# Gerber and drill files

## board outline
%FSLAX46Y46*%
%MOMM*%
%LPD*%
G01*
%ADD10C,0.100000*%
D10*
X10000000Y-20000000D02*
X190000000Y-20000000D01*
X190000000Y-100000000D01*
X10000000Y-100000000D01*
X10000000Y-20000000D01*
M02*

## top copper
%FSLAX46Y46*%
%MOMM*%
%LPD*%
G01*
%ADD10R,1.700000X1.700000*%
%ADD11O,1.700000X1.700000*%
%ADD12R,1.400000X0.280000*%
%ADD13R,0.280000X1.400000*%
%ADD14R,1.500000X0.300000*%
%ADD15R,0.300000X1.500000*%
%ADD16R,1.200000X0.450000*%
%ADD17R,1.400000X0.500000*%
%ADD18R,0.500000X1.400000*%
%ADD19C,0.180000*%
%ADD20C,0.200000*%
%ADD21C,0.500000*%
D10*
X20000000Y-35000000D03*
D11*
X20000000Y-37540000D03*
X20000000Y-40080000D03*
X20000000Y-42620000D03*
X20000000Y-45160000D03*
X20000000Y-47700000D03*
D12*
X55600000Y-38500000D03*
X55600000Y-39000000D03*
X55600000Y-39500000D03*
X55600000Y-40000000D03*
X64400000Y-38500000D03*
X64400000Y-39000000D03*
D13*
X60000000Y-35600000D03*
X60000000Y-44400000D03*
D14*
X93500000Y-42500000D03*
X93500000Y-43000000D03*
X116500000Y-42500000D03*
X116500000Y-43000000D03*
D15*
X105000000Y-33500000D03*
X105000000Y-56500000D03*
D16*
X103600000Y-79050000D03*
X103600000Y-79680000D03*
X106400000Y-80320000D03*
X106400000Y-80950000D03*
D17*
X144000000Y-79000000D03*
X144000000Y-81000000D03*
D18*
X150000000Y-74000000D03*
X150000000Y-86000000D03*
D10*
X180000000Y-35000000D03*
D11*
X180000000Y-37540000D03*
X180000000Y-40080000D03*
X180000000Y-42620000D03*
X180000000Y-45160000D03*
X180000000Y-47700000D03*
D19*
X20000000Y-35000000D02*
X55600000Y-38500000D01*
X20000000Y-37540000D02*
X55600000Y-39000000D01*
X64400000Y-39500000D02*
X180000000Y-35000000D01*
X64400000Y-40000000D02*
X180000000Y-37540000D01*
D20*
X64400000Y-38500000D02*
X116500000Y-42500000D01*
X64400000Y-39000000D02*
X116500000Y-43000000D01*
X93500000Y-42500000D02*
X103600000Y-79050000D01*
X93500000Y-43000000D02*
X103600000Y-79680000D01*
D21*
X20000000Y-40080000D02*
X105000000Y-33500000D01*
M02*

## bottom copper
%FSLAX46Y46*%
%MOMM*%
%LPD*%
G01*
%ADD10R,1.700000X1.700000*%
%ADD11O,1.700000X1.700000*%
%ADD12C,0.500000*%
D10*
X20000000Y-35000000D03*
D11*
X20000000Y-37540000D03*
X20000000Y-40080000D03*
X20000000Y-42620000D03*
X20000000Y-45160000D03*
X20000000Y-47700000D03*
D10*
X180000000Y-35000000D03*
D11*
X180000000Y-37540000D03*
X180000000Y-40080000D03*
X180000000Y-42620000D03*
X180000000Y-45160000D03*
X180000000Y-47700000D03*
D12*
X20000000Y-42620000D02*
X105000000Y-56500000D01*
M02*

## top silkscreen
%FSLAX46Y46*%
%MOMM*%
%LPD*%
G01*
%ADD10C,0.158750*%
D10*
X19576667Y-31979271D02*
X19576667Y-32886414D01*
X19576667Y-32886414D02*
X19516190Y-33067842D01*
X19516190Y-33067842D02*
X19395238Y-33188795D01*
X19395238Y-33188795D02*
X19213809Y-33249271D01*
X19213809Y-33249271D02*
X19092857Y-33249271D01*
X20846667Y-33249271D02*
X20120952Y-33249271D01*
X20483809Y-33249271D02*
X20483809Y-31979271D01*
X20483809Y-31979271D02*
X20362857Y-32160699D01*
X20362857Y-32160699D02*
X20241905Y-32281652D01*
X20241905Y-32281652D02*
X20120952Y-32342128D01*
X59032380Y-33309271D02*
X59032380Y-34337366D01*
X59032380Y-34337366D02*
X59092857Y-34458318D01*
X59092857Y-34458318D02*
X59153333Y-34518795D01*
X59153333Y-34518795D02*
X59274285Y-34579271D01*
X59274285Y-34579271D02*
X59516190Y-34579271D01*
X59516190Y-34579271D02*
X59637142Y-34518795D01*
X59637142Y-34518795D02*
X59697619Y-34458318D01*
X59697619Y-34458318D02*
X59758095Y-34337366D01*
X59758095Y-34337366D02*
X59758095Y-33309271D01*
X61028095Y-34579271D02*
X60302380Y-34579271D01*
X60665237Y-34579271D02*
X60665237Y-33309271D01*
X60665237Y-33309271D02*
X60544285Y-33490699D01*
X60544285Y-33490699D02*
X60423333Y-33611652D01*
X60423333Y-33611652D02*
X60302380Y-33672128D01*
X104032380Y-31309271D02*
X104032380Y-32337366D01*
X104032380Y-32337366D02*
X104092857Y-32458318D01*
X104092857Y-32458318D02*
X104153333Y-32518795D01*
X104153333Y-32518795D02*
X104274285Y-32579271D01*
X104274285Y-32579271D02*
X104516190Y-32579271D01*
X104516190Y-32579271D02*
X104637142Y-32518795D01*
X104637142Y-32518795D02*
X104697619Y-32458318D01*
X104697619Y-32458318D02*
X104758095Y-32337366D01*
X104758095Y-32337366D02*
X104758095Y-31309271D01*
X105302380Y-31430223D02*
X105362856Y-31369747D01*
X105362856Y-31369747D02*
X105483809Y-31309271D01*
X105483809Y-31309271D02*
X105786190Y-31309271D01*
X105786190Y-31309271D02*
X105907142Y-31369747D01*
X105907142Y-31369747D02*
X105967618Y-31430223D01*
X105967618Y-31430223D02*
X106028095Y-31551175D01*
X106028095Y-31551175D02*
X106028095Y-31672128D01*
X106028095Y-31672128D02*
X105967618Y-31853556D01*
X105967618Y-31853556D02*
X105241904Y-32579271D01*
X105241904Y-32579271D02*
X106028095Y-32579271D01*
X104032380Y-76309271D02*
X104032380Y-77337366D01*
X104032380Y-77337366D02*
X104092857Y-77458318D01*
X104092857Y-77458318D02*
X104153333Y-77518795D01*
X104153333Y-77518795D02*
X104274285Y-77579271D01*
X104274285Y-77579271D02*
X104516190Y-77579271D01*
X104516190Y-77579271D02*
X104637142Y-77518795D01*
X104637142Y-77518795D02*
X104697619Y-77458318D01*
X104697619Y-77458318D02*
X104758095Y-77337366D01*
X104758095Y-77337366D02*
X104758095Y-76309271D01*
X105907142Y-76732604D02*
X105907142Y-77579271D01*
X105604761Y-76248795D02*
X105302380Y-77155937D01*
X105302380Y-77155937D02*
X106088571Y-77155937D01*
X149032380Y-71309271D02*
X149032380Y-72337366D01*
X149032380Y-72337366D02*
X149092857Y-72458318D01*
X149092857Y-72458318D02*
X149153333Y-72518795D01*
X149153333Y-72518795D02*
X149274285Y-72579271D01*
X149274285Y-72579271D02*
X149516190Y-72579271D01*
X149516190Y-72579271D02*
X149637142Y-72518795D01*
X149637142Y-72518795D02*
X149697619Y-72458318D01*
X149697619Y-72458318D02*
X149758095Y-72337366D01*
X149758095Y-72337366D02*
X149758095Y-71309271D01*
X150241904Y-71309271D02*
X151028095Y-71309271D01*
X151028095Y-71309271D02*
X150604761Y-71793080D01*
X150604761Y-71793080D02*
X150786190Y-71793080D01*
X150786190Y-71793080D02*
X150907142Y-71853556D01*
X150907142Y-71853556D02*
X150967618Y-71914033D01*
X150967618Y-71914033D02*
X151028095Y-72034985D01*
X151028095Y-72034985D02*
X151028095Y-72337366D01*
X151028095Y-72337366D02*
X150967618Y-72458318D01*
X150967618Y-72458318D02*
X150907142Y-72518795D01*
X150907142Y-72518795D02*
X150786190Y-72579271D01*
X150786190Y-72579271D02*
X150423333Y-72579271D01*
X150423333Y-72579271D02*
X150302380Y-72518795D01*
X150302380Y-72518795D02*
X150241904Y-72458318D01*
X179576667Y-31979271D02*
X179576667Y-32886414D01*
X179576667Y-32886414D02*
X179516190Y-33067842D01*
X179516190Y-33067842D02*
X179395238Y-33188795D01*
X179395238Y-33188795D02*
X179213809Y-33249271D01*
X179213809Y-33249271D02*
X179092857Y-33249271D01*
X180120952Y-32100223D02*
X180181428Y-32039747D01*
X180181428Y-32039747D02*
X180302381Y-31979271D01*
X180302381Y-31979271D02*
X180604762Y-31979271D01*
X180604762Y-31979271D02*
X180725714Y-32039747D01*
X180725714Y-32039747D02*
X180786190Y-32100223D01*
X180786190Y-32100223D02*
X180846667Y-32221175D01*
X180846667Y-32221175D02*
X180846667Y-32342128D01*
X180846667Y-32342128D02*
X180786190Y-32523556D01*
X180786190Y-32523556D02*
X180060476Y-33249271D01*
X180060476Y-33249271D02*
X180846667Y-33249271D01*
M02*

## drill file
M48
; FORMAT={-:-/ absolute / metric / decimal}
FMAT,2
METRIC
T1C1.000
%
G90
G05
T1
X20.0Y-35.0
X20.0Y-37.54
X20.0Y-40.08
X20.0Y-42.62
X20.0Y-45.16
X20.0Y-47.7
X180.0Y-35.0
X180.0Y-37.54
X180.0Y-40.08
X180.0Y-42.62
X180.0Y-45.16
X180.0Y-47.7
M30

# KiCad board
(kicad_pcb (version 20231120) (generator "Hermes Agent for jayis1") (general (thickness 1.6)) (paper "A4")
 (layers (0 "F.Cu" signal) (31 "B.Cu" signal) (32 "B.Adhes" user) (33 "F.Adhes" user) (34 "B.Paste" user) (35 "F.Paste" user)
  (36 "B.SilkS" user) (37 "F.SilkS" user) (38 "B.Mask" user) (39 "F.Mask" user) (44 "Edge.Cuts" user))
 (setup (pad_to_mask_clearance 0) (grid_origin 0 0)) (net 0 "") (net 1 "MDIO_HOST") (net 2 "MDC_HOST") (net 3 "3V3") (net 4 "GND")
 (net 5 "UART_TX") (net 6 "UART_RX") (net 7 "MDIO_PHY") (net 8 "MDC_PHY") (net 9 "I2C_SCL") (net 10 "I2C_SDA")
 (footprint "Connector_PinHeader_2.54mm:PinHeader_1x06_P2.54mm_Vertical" (layer "F.Cu") (at 20 35)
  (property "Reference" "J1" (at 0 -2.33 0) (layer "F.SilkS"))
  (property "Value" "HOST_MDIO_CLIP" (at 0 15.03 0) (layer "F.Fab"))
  (pad "1" thru_hole rect (at 0 0) (size 1.7 1.7) (drill 1) (layers "*.Cu" "*.Mask") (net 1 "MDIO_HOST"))
  (pad "2" thru_hole oval (at 0 2.54) (size 1.7 1.7) (drill 1) (layers "*.Cu" "*.Mask") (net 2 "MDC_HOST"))
  (pad "3" thru_hole oval (at 0 5.08) (size 1.7 1.7) (drill 1) (layers "*.Cu" "*.Mask") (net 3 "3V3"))
  (pad "4" thru_hole oval (at 0 7.62) (size 1.7 1.7) (drill 1) (layers "*.Cu" "*.Mask") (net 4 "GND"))
  (pad "5" thru_hole oval (at 0 10.16) (size 1.7 1.7) (drill 1) (layers "*.Cu" "*.Mask") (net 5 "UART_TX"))
  (pad "6" thru_hole oval (at 0 12.70) (size 1.7 1.7) (drill 1) (layers "*.Cu" "*.Mask") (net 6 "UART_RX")))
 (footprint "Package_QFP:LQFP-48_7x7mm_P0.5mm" (layer "F.Cu") (at 60 40) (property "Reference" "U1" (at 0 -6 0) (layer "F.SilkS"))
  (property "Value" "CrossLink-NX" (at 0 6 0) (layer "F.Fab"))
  (pad "5" smd rect (at -4.4 -1.5) (size 1.4 0.28) (layers "F.Cu" "F.Paste" "F.Mask") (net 1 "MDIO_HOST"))
  (pad "6" smd rect (at -4.4 -1.0) (size 1.4 0.28) (layers "F.Cu" "F.Paste" "F.Mask") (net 2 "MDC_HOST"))
  (pad "7" smd rect (at -4.4 -0.5) (size 1.4 0.28) (layers "F.Cu" "F.Paste" "F.Mask") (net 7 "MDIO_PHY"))
  (pad "8" smd rect (at -4.4 0.0) (size 1.4 0.28) (layers "F.Cu" "F.Paste" "F.Mask") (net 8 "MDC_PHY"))
  (pad "44" smd rect (at 4.4 -1.5) (size 1.4 0.28) (layers "F.Cu" "F.Paste" "F.Mask") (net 5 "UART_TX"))
  (pad "45" smd rect (at 4.4 -1.0) (size 1.4 0.28) (layers "F.Cu" "F.Paste" "F.Mask") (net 6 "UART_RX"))
  (pad "62" smd rect (at 0 -4.4) (size 0.28 1.4) (layers "F.Cu" "F.Paste" "F.Mask") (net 3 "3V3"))
  (pad "31" smd rect (at 0 4.4) (size 0.28 1.4) (layers "F.Cu" "F.Paste" "F.Mask") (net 4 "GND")))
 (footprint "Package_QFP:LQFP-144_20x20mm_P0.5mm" (layer "F.Cu") (at 105 45) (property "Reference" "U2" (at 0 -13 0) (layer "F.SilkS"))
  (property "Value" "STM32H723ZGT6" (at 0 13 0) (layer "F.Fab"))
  (pad "95" smd rect (at -11.5 -2.5) (size 1.5 0.3) (layers "F.Cu" "F.Paste" "F.Mask") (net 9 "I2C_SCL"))
  (pad "96" smd rect (at -11.5 -2.0) (size 1.5 0.3) (layers "F.Cu" "F.Paste" "F.Mask") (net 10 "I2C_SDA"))
  (pad "51" smd rect (at 11.5 -2.5) (size 1.5 0.3) (layers "F.Cu" "F.Paste" "F.Mask") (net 5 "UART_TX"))
  (pad "52" smd rect (at 11.5 -2.0) (size 1.5 0.3) (layers "F.Cu" "F.Paste" "F.Mask") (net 6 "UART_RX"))
  (pad "13" smd rect (at 0 -11.5) (size 0.3 1.5) (layers "F.Cu" "F.Paste" "F.Mask") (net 3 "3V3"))
  (pad "64" smd rect (at 0 11.5) (size 0.3 1.5) (layers "F.Cu" "F.Paste" "F.Mask") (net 4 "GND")))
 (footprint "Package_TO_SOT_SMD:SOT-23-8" (layer "F.Cu") (at 105 80) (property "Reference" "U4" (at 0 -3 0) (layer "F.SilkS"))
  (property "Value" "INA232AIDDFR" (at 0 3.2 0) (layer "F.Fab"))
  (pad "1" smd rect (at -1.4 -0.95) (size 1.2 0.45) (layers "F.Cu" "F.Paste" "F.Mask") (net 9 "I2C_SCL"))
  (pad "2" smd rect (at -1.4 -0.32) (size 1.2 0.45) (layers "F.Cu" "F.Paste" "F.Mask") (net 10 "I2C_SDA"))
  (pad "6" smd rect (at 1.4 0.32) (size 1.2 0.45) (layers "F.Cu" "F.Paste" "F.Mask") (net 3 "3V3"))
  (pad "5" smd rect (at 1.4 0.95) (size 1.2 0.45) (layers "F.Cu" "F.Paste" "F.Mask") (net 4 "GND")))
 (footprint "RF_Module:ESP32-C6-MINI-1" (layer "F.Cu") (at 150 80) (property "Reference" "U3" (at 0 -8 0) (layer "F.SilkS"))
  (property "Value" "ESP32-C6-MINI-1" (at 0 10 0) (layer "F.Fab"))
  (pad "30" smd rect (at -6 -1) (size 1.4 0.5) (layers "F.Cu" "F.Paste" "F.Mask") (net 5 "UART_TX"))
  (pad "31" smd rect (at -6 1) (size 1.4 0.5) (layers "F.Cu" "F.Paste" "F.Mask") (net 6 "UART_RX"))
  (pad "1" smd rect (at 0 -6) (size 0.5 1.4) (layers "F.Cu" "F.Paste" "F.Mask") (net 3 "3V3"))
  (pad "15" smd rect (at 0 6) (size 0.5 1.4) (layers "F.Cu" "F.Paste" "F.Mask") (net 4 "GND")))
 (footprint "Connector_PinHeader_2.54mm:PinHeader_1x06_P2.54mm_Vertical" (layer "F.Cu") (at 180 35)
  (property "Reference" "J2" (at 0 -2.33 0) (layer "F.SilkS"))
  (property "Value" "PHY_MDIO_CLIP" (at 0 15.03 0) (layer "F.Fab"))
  (pad "1" thru_hole rect (at 0 0) (size 1.7 1.7) (drill 1) (layers "*.Cu" "*.Mask") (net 7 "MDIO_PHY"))
  (pad "2" thru_hole oval (at 0 2.54) (size 1.7 1.7) (drill 1) (layers "*.Cu" "*.Mask") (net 8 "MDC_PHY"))
  (pad "3" thru_hole oval (at 0 5.08) (size 1.7 1.7) (drill 1) (layers "*.Cu" "*.Mask") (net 3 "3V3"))
  (pad "4" thru_hole oval (at 0 7.62) (size 1.7 1.7) (drill 1) (layers "*.Cu" "*.Mask") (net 4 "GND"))
  (pad "5" thru_hole oval (at 0 10.16) (size 1.7 1.7) (drill 1) (layers "*.Cu" "*.Mask") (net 9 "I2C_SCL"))
  (pad "6" thru_hole oval (at 0 12.70) (size 1.7 1.7) (drill 1) (layers "*.Cu" "*.Mask") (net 10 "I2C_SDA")))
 (segment (start 20 35) (end 55.6 38.5) (width 0.18) (layer "F.Cu") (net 1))
 (segment (start 20 37.54) (end 55.6 39.0) (width 0.18) (layer "F.Cu") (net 2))
 (segment (start 64.4 39.5) (end 180 35) (width 0.18) (layer "F.Cu") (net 7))
 (segment (start 64.4 40.0) (end 180 37.54) (width 0.18) (layer "F.Cu") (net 8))
 (segment (start 64.4 38.5) (end 116.5 42.5) (width 0.2) (layer "F.Cu") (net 5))
 (segment (start 64.4 39.0) (end 116.5 43.0) (width 0.2) (layer "F.Cu") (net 6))
 (segment (start 93.5 42.5) (end 103.6 79.05) (width 0.2) (layer "F.Cu") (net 9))
 (segment (start 93.5 43.0) (end 103.6 79.68) (width 0.2) (layer "F.Cu") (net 10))
 (segment (start 20 40.08) (end 105 33.5) (width 0.5) (layer "F.Cu") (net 3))
 (segment (start 20 42.62) (end 105 56.5) (width 0.5) (layer "B.Cu") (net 4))
 (gr_rect (start 10 20) (end 190 100) (stroke (width 0.1) (type default)) (fill none) (layer "Edge.Cuts")))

